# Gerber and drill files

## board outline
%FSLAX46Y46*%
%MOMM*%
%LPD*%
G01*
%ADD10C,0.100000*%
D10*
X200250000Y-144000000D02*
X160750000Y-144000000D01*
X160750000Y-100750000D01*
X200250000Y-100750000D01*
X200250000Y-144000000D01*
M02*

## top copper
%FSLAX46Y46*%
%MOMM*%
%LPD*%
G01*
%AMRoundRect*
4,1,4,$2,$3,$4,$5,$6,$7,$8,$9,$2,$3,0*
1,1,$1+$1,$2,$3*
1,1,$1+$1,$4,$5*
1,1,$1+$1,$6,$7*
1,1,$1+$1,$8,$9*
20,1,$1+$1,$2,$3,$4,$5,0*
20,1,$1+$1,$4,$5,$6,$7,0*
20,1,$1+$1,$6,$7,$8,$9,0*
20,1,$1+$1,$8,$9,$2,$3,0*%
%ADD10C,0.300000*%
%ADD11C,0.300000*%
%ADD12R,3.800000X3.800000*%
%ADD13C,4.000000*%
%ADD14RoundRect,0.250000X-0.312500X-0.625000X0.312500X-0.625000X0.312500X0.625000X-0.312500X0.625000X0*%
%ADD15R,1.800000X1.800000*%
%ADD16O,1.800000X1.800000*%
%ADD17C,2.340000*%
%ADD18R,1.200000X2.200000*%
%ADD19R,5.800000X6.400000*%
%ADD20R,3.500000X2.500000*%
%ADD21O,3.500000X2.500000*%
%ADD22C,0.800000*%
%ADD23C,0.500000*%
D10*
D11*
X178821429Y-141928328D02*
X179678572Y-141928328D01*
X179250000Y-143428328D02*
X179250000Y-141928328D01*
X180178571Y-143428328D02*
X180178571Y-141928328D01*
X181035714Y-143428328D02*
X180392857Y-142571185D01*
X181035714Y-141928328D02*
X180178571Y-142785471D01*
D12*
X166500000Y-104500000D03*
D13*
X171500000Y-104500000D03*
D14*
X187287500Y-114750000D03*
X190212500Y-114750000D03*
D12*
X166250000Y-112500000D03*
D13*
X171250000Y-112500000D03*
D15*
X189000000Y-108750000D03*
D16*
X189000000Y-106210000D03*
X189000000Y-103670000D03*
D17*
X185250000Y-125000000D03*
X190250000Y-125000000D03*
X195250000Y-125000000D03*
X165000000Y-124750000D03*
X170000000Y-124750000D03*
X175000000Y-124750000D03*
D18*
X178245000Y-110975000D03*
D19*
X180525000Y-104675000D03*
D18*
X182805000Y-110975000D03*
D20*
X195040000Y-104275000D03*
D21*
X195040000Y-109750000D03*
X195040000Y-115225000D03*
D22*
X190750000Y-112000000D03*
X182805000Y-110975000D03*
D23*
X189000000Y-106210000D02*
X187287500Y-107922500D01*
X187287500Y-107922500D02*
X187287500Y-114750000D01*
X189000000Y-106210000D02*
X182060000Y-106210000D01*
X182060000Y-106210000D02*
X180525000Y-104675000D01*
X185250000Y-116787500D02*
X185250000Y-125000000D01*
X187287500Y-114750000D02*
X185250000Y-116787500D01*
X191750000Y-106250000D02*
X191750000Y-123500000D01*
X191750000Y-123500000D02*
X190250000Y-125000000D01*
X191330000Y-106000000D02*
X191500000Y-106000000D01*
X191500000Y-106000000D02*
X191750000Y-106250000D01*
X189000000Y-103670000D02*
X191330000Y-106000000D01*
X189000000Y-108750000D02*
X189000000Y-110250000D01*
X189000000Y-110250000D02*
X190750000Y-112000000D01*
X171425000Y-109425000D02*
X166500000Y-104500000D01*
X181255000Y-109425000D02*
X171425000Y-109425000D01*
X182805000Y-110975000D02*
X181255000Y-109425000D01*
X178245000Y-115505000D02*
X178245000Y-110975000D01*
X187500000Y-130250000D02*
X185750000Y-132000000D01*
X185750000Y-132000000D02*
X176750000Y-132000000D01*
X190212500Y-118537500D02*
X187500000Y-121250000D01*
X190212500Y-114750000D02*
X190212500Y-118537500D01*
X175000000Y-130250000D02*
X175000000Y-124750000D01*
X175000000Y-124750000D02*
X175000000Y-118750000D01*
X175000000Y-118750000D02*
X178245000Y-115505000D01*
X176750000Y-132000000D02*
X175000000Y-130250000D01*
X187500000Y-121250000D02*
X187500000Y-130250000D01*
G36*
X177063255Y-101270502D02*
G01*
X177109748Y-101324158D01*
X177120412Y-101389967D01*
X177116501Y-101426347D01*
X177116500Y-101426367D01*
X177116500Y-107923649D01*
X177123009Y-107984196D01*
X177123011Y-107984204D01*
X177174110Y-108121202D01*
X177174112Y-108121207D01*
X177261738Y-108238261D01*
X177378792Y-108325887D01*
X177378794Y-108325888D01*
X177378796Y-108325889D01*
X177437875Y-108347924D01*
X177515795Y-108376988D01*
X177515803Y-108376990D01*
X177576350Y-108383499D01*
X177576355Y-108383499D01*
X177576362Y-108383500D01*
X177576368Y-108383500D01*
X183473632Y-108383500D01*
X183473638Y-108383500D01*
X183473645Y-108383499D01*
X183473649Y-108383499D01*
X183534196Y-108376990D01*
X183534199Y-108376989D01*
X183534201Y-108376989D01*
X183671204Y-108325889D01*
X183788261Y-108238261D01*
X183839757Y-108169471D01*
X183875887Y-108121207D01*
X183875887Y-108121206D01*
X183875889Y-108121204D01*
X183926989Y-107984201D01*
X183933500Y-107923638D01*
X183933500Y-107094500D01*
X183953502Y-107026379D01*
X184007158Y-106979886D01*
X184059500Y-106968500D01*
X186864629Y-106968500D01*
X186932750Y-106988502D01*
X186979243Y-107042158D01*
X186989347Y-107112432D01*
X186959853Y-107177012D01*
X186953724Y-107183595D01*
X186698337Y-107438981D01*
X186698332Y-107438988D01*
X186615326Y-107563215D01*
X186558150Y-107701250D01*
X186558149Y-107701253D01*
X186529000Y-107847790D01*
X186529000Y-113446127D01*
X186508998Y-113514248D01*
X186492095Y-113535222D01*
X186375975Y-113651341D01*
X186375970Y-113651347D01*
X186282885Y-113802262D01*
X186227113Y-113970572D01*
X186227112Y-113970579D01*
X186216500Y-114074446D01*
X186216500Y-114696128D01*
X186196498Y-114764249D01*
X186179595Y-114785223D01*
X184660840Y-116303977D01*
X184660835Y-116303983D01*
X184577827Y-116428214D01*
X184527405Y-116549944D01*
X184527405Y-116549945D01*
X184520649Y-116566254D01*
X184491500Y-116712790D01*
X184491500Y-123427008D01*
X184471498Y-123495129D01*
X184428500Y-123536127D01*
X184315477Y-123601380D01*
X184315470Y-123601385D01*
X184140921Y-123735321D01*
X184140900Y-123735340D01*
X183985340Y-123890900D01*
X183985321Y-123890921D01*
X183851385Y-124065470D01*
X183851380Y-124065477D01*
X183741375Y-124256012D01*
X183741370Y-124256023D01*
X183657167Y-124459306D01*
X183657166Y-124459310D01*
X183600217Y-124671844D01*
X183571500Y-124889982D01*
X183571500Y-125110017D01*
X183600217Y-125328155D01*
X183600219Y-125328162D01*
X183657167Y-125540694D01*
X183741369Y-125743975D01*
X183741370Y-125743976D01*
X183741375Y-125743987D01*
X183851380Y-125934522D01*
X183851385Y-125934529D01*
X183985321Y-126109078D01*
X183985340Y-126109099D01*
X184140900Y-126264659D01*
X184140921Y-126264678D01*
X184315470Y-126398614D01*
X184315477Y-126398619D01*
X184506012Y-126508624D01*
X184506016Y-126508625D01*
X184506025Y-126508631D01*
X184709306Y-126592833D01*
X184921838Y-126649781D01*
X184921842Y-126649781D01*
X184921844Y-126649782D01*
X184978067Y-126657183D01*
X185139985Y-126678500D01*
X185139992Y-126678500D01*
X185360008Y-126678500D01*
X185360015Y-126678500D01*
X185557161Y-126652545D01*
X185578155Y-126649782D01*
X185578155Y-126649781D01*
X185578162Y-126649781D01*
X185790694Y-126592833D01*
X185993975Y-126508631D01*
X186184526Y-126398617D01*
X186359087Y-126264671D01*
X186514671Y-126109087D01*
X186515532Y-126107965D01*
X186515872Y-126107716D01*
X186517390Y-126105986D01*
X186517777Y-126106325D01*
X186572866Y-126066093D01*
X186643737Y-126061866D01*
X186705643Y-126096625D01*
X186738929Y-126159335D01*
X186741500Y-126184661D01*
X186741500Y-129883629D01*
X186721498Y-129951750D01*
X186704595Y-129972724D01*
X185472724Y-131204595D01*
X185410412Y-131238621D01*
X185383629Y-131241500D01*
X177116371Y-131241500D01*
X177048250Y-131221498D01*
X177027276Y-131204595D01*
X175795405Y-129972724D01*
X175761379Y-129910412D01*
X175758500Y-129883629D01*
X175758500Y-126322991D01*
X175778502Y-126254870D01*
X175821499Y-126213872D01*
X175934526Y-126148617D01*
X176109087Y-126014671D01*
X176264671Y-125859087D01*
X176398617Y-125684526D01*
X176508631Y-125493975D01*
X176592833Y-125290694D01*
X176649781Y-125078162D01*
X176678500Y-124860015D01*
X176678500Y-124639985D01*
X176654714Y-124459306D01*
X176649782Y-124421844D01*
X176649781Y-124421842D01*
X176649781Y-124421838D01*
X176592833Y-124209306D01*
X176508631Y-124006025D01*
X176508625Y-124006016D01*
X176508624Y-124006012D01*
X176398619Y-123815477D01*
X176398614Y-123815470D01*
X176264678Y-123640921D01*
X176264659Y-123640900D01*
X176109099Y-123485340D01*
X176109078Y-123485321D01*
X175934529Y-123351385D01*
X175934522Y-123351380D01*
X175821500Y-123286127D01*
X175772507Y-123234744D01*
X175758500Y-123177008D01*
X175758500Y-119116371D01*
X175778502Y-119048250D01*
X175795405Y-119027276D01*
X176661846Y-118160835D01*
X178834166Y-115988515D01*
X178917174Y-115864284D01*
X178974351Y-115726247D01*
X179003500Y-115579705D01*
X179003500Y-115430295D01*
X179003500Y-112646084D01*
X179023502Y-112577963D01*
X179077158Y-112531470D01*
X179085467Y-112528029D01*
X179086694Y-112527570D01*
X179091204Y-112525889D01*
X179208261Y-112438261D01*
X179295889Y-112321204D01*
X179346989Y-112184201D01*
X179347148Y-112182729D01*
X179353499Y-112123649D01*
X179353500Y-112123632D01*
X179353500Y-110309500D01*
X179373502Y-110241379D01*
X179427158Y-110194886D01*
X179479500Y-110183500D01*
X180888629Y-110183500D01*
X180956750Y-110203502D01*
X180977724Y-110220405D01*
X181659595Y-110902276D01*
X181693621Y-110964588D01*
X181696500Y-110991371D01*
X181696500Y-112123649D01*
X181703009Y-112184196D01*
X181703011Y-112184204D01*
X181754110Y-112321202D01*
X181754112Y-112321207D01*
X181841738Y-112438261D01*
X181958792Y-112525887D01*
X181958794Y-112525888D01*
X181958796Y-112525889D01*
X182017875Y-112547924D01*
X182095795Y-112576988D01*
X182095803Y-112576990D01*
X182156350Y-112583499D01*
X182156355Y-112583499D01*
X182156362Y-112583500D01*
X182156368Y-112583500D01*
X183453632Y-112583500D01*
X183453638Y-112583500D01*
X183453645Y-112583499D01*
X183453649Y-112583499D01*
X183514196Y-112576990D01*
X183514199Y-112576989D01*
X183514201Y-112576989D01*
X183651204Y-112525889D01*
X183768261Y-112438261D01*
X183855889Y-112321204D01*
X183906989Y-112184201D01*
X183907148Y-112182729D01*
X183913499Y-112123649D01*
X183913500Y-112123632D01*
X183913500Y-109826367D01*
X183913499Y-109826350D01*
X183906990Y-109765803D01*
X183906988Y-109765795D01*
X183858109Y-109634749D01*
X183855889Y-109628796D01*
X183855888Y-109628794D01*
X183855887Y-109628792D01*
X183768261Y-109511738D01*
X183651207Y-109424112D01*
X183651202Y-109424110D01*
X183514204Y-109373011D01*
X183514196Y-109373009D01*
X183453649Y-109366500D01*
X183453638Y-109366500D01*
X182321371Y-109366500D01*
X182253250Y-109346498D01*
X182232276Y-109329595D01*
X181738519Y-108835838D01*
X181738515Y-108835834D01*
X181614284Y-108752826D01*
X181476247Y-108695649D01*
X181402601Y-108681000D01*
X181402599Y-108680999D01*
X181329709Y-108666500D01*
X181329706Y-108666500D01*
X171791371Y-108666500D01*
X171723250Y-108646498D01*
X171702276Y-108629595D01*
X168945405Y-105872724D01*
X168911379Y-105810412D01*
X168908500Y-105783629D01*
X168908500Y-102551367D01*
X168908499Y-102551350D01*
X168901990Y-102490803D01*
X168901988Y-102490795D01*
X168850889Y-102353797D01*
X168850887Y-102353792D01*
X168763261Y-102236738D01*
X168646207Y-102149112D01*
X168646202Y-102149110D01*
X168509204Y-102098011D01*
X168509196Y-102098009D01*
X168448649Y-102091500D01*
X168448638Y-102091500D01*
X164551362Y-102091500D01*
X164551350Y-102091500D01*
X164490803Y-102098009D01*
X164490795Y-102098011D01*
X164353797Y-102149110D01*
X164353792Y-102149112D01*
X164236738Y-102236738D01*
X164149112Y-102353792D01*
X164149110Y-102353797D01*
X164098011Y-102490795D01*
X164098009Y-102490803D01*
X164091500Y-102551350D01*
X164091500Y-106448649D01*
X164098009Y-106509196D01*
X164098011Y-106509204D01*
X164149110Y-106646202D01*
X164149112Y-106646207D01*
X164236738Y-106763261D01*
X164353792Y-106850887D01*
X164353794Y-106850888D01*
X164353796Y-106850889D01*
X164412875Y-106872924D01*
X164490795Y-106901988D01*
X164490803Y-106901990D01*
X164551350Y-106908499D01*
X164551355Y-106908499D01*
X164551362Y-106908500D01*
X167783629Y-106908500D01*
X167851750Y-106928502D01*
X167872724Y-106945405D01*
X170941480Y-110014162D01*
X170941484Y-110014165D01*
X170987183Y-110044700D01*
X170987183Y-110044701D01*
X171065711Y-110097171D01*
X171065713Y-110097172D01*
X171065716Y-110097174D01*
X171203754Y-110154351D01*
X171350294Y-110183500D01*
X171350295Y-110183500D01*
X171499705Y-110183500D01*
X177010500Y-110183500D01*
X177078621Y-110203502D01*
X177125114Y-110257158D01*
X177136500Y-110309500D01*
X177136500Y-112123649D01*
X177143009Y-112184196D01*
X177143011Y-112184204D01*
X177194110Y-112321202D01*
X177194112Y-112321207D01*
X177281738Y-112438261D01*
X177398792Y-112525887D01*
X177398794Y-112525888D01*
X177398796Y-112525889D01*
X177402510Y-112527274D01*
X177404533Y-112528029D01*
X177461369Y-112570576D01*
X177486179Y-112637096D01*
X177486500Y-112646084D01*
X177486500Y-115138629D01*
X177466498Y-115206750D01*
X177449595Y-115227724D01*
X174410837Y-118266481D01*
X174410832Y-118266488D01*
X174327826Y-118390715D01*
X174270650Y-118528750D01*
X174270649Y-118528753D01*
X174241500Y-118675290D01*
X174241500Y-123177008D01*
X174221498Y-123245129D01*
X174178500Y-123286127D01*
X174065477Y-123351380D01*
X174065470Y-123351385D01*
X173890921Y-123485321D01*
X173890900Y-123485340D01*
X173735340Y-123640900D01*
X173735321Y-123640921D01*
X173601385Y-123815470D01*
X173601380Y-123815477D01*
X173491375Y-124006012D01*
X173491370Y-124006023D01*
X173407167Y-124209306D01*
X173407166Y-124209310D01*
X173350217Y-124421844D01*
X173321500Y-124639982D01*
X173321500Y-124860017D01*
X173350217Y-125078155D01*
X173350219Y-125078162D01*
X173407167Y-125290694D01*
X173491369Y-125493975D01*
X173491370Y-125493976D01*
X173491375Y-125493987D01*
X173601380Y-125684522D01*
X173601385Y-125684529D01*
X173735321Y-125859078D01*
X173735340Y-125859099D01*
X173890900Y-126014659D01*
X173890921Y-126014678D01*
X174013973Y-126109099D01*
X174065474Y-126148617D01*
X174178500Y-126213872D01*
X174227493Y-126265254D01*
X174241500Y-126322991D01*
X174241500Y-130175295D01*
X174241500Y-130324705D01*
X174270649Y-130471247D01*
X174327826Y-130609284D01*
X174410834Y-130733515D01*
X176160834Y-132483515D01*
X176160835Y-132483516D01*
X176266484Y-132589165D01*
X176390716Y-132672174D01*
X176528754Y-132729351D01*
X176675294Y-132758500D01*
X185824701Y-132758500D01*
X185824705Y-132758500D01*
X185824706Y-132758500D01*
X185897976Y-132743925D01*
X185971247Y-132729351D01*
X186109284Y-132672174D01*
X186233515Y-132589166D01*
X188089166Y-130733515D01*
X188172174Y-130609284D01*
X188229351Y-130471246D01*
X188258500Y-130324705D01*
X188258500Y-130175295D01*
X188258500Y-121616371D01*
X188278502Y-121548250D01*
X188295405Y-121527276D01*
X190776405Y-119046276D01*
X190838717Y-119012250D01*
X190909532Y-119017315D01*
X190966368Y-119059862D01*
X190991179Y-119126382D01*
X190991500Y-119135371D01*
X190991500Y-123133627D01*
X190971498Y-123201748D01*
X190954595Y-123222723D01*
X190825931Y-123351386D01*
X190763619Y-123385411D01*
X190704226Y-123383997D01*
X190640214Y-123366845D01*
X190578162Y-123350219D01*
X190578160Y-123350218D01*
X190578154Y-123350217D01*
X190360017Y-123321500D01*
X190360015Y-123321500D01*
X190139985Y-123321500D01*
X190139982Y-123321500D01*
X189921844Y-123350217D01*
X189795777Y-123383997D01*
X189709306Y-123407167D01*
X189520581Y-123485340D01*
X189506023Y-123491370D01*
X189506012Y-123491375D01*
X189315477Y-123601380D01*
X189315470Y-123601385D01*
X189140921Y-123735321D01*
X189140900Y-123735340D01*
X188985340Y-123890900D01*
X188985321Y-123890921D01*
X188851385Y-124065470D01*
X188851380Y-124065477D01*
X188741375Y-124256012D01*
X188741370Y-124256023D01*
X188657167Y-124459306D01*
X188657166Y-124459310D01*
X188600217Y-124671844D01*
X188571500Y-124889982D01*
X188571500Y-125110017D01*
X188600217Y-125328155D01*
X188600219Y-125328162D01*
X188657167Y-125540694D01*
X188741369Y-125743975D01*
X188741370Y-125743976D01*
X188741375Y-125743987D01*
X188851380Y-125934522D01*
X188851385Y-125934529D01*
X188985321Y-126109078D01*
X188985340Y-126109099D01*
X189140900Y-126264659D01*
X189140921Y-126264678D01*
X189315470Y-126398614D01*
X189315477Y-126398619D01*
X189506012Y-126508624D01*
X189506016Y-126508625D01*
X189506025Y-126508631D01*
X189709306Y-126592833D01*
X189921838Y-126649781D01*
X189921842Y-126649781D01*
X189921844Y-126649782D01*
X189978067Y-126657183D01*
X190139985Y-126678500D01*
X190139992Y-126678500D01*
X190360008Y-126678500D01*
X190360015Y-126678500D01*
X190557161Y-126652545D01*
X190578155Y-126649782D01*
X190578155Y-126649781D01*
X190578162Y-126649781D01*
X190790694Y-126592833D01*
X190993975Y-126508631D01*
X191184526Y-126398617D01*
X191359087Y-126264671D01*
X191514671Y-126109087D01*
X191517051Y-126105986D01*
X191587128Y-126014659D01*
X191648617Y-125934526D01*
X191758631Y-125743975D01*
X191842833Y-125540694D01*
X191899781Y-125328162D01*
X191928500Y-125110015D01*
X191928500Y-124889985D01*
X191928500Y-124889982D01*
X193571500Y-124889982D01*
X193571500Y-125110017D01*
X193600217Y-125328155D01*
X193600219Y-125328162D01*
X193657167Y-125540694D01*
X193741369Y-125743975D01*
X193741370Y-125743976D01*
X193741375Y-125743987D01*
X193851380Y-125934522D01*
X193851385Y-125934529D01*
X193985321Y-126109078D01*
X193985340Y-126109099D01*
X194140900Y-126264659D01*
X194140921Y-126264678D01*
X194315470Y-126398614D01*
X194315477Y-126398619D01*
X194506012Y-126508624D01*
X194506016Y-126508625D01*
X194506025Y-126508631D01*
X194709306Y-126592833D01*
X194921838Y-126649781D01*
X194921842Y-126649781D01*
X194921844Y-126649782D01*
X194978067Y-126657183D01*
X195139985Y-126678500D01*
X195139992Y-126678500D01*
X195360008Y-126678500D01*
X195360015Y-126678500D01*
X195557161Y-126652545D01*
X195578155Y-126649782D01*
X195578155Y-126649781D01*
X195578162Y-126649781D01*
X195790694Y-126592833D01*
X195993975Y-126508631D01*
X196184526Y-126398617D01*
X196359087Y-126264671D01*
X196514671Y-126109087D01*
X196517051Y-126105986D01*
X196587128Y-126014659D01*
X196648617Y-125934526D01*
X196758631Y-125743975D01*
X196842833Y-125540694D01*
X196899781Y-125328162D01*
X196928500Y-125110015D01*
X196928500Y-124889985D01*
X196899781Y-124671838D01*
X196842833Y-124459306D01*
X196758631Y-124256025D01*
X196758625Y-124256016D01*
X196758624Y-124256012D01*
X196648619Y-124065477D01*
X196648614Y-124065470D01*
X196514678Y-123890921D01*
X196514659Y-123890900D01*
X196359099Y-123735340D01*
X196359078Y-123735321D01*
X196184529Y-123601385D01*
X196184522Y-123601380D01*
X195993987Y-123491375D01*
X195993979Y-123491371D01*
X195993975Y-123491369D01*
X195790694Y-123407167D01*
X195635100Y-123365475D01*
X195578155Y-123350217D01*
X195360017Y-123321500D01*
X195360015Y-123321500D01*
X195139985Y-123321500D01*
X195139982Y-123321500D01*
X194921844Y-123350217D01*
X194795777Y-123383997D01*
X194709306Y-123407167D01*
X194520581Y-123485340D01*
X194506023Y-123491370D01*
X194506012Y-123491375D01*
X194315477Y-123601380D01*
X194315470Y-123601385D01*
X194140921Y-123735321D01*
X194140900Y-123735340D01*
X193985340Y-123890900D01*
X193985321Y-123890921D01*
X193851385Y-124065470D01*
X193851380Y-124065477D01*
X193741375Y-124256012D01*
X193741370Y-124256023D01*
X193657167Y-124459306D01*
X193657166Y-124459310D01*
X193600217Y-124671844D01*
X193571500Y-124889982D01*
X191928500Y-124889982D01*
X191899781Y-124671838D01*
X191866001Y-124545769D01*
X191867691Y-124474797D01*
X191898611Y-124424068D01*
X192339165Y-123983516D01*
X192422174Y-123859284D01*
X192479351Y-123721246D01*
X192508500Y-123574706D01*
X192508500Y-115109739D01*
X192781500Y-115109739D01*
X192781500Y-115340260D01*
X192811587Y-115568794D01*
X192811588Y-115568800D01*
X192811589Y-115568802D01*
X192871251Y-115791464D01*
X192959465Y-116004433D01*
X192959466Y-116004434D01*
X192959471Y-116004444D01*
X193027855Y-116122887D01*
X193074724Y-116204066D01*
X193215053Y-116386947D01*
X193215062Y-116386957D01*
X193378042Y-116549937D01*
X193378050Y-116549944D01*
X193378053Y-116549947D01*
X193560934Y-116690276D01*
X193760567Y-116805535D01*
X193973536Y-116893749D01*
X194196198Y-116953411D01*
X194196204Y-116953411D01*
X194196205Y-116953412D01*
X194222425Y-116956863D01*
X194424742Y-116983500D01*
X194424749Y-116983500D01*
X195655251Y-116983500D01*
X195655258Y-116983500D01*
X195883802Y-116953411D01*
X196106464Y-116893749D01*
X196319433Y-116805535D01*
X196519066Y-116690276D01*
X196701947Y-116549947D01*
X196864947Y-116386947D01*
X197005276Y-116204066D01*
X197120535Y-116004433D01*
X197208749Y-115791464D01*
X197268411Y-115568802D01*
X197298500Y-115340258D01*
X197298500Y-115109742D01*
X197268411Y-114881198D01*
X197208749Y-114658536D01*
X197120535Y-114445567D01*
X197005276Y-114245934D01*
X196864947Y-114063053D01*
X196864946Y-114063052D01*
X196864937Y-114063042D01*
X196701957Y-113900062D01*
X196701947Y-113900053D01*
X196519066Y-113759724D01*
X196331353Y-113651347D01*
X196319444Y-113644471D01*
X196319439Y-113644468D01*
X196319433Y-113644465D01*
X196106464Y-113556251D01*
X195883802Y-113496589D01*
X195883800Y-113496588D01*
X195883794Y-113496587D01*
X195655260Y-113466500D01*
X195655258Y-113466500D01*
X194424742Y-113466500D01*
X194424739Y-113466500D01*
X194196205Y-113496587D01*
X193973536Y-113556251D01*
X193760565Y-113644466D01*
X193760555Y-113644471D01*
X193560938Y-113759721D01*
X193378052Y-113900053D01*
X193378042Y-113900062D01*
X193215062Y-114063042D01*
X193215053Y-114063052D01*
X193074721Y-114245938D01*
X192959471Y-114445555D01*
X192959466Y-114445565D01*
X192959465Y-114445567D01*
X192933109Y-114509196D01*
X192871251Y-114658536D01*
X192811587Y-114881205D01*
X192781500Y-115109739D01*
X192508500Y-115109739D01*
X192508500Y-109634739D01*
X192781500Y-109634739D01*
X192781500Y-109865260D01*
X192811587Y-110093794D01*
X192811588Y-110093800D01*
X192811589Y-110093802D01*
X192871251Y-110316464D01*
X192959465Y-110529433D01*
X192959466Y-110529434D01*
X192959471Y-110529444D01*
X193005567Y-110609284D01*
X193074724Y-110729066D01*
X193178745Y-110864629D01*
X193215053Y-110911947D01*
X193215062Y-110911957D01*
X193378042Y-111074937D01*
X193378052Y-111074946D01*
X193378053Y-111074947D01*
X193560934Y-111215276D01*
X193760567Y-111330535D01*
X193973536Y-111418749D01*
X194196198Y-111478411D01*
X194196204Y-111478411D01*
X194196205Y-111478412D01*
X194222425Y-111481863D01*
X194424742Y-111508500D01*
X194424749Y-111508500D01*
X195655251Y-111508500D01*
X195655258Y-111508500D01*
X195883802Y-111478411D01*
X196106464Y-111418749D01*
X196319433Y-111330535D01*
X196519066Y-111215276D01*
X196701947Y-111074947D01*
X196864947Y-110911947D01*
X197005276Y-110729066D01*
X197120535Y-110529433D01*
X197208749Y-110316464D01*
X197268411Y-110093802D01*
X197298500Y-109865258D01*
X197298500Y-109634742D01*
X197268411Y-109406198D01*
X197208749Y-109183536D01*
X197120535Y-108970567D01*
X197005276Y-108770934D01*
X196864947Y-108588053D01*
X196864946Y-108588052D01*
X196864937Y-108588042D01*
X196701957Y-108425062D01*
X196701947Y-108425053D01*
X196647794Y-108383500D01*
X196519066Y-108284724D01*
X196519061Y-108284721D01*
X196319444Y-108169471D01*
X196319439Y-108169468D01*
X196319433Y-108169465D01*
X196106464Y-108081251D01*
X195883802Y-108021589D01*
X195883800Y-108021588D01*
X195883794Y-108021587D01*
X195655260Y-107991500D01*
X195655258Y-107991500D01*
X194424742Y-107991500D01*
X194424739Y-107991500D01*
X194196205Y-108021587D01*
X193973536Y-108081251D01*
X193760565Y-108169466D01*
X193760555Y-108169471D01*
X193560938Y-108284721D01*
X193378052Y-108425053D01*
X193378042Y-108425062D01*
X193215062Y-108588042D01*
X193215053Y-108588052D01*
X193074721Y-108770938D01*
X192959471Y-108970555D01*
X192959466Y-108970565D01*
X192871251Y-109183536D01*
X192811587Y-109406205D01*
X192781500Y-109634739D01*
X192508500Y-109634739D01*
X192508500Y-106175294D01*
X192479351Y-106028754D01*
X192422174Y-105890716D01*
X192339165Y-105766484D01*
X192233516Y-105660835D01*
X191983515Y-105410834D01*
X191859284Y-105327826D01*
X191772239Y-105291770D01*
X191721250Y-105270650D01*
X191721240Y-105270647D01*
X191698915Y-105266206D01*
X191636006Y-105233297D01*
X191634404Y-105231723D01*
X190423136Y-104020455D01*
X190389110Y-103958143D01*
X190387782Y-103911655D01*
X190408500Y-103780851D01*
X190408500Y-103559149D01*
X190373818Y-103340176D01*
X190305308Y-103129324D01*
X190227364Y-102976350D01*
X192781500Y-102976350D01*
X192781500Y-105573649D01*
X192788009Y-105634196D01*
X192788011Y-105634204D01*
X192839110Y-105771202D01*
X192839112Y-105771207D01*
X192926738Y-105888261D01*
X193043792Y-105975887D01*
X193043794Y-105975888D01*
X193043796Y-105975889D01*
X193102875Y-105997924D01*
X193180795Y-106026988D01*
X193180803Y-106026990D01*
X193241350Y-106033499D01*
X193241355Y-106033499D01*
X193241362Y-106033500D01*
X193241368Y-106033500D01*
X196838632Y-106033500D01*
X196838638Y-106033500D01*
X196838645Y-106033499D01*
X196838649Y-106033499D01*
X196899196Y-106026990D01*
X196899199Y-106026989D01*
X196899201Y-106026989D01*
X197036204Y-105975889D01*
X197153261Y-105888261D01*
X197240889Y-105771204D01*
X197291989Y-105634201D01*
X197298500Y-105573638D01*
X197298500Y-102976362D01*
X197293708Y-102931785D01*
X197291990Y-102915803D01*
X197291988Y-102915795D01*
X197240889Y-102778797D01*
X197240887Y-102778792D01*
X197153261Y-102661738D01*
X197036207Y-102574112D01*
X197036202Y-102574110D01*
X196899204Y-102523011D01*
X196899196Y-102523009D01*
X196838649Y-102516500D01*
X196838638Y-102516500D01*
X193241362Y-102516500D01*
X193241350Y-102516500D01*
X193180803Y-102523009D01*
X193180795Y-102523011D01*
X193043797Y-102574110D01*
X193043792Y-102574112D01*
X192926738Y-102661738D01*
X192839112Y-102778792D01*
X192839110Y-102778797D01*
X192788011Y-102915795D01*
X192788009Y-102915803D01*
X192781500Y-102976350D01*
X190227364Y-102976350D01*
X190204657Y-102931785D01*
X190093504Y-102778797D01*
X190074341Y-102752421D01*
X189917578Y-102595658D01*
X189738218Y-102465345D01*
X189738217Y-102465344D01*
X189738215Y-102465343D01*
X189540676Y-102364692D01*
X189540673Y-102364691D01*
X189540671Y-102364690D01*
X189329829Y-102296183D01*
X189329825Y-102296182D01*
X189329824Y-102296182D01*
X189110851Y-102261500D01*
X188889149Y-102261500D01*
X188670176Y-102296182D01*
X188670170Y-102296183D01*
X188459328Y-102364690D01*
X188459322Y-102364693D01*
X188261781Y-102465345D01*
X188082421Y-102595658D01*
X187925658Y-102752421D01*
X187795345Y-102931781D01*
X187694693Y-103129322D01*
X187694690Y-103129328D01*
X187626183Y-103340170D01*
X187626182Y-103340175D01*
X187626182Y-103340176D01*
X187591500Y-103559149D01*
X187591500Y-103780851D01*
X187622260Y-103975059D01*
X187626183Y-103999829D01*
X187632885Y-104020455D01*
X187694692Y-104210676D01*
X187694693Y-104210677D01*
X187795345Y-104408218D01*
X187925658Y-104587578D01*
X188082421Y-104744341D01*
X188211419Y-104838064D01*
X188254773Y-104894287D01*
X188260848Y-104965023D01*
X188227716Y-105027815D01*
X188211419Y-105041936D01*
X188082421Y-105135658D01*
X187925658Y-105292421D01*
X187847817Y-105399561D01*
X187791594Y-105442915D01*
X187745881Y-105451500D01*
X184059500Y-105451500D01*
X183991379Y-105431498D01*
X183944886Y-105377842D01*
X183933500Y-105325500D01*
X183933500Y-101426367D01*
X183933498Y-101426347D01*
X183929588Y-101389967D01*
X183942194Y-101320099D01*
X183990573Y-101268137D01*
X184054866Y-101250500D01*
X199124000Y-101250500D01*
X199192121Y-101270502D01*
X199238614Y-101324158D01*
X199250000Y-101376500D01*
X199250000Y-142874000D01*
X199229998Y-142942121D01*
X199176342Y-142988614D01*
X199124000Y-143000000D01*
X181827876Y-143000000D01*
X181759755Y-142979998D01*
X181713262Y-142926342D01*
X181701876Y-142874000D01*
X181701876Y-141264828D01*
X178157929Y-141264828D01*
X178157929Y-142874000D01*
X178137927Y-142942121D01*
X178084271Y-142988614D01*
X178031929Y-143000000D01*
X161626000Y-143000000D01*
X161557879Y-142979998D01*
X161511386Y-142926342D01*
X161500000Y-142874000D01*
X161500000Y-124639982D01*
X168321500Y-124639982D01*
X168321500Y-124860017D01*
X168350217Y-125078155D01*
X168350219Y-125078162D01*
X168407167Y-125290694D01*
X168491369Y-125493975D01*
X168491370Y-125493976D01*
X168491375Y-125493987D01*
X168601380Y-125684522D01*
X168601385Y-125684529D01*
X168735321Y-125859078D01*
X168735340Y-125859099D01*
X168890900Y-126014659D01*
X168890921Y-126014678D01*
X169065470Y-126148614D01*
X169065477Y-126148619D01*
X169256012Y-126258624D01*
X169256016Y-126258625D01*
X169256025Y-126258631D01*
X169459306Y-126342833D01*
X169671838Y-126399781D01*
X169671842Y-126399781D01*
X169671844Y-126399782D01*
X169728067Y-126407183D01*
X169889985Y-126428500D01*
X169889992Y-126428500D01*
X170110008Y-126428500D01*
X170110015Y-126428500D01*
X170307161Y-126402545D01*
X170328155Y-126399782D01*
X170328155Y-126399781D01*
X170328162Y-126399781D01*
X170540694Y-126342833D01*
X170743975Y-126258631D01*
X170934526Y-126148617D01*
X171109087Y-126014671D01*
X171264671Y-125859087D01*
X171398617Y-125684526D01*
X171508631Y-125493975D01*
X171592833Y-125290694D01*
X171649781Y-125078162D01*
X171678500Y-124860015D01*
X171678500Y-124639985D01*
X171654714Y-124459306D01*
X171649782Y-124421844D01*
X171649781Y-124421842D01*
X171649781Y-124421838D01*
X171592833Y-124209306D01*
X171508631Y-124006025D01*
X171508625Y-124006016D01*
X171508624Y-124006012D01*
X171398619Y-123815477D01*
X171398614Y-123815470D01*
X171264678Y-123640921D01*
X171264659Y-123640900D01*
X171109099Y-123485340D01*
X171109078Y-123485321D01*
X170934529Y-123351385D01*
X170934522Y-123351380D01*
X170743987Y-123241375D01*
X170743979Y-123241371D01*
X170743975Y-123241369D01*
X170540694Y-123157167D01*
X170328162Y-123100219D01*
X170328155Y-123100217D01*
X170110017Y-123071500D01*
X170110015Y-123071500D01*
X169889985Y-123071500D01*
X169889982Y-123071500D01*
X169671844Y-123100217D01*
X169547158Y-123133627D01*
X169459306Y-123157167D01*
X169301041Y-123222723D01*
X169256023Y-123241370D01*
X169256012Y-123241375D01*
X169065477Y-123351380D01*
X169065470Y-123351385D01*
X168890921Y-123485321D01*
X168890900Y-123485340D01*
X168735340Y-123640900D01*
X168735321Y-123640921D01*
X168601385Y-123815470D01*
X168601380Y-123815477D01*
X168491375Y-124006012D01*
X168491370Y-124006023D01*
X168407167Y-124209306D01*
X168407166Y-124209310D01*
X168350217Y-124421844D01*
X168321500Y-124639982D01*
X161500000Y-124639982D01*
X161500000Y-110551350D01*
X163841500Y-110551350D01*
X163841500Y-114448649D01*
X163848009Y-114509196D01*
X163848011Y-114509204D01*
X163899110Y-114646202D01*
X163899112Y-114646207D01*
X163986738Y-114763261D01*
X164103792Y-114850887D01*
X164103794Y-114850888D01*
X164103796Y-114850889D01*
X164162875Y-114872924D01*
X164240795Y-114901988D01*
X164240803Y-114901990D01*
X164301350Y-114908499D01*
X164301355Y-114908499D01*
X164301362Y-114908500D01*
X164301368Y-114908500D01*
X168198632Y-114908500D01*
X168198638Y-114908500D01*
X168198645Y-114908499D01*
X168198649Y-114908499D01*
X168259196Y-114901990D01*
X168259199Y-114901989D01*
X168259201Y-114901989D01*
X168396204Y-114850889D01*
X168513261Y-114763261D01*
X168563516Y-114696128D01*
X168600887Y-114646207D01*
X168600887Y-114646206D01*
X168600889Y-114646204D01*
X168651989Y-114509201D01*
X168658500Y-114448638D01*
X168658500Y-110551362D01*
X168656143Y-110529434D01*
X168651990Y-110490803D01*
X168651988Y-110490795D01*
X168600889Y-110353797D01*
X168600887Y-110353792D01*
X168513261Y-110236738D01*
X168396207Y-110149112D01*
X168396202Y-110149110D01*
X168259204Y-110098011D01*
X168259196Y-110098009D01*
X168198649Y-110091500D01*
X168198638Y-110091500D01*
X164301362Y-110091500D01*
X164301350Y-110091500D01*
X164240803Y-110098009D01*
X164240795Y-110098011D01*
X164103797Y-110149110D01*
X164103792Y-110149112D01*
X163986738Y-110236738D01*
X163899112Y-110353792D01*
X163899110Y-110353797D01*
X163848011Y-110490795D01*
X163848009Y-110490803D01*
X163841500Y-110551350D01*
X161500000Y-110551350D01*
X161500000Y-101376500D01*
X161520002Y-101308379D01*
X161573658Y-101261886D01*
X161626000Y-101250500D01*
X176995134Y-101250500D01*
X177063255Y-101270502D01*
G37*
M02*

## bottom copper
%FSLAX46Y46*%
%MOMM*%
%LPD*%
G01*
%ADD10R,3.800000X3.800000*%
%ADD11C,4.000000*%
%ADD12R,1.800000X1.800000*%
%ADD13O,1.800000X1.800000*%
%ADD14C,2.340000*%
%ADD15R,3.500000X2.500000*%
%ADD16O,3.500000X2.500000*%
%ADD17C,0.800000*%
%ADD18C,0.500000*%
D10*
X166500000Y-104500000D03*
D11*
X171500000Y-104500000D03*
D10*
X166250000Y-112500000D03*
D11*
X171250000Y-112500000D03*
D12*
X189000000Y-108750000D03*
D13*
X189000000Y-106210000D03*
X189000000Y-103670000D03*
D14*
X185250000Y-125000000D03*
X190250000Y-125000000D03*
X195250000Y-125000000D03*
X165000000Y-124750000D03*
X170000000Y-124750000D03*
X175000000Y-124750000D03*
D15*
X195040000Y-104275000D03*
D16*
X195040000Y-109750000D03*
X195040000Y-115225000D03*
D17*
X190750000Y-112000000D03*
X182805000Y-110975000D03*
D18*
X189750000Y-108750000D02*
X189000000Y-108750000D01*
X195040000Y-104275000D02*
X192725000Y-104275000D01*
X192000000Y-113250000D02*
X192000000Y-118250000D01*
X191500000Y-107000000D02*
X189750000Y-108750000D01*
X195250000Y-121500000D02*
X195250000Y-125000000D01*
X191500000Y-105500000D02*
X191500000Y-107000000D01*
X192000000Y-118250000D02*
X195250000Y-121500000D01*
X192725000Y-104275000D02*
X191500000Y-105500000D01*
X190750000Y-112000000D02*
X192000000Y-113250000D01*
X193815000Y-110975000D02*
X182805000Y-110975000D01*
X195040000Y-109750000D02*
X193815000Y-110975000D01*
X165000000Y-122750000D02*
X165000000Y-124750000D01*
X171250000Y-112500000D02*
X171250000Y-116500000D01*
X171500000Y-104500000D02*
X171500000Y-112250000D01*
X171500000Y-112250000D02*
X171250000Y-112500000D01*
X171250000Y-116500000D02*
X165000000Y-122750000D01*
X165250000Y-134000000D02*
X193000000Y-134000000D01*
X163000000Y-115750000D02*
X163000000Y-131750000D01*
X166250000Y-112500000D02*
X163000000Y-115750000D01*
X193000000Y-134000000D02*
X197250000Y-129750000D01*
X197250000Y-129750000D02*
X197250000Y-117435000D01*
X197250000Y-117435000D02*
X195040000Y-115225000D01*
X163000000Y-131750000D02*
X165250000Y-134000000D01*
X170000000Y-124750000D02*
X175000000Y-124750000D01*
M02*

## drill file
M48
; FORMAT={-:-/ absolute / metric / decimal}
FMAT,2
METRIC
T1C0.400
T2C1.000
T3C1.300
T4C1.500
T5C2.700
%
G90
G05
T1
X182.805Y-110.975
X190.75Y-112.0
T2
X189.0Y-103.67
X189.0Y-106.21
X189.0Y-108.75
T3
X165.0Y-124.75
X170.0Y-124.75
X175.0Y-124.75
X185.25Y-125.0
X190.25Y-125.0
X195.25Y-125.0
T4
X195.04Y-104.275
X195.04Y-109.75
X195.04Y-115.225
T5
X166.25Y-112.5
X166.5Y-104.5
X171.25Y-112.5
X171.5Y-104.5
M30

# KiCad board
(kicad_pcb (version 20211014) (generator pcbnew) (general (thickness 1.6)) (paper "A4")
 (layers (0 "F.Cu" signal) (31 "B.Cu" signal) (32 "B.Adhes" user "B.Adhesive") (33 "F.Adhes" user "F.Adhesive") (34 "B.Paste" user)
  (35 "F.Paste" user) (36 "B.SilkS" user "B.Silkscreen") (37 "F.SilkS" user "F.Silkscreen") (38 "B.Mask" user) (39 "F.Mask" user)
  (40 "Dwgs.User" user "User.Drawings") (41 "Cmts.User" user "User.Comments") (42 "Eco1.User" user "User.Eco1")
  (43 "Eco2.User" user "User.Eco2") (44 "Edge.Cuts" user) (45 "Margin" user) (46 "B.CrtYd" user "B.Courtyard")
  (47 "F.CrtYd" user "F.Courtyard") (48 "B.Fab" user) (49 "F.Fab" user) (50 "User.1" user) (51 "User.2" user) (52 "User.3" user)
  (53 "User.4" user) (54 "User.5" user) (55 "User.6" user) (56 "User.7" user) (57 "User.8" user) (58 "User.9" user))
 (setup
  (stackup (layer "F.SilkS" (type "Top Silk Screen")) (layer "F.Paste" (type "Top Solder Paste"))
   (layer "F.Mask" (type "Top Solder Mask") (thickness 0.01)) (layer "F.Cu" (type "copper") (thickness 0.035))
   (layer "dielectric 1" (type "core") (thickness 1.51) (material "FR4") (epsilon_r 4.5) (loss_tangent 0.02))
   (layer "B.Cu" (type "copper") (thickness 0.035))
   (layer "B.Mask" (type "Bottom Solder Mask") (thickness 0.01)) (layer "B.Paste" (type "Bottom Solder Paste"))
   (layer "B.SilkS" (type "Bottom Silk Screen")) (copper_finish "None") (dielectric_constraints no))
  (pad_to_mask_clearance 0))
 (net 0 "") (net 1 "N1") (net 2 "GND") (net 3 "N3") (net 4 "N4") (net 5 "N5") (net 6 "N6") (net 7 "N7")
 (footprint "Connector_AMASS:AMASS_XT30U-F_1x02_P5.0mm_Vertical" (layer "F.Cu") (at 166.5 104.5)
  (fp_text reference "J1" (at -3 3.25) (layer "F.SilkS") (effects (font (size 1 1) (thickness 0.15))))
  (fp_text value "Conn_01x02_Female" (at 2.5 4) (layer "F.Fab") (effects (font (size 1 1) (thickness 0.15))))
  (pad "1" thru_hole rect (at 0 0) (size 3.8 3.8) (drill 2.7) (layers *.Cu *.Mask) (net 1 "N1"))
  (pad "2" thru_hole circle (at 5 0) (size 4 4) (drill 2.7) (layers *.Cu *.Mask) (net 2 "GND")))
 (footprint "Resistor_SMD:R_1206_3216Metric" (layer "F.Cu") (at 188.75 114.75)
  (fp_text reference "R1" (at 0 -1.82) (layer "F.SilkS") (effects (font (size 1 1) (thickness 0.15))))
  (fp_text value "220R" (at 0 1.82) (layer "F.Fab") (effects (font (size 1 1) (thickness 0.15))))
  (pad "1" smd roundrect (at -1.4625 0) (size 1.125 1.75) (layers "F.Cu" "F.Paste" "F.Mask") (roundrect_rratio 0.2222222222) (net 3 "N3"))
  (pad "2" smd roundrect (at 1.4625 0) (size 1.125 1.75) (layers "F.Cu" "F.Paste" "F.Mask") (roundrect_rratio 0.2222222222) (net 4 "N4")))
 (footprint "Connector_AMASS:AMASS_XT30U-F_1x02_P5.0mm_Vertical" (layer "F.Cu") (at 166.25 112.5)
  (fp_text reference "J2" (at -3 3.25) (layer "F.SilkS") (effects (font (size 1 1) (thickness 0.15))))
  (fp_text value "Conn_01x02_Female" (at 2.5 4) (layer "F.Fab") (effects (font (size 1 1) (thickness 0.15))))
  (pad "1" thru_hole rect (at 0 0) (size 3.8 3.8) (drill 2.7) (layers *.Cu *.Mask) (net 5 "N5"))
  (pad "2" thru_hole circle (at 5 0) (size 4 4) (drill 2.7) (layers *.Cu *.Mask) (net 2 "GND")))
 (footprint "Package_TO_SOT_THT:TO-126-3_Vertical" (layer "F.Cu") (at 189 108.75 90)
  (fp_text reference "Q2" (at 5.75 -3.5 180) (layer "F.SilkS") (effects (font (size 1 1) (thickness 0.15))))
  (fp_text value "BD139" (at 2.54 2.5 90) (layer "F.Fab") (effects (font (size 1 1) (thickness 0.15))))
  (pad "1" thru_hole rect (at 0 0 90) (size 1.8 1.8) (drill 1) (layers *.Cu *.Mask) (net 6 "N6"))
  (pad "2" thru_hole oval (at 2.54 0 90) (size 1.8 1.8) (drill 1) (layers *.Cu *.Mask) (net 3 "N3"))
  (pad "3" thru_hole oval (at 5.08 0 90) (size 1.8 1.8) (drill 1) (layers *.Cu *.Mask) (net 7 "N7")))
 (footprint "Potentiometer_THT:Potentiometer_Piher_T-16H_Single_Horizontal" (layer "F.Cu") (at 185.25 125 -90)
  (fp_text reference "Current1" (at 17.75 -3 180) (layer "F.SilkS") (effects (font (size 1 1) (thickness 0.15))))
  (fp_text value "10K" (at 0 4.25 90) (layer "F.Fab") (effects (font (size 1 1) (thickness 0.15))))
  (pad "1" thru_hole circle (at 0 0 270) (size 2.34 2.34) (drill 1.3) (layers *.Cu *.Mask) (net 3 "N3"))
  (pad "2" thru_hole circle (at 0 -5 270) (size 2.34 2.34) (drill 1.3) (layers *.Cu *.Mask) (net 7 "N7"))
  (pad "3" thru_hole circle (at 0 -10 270) (size 2.34 2.34) (drill 1.3) (layers *.Cu *.Mask) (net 6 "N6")))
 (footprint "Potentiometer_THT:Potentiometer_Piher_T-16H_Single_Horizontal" (layer "F.Cu") (at 165 124.75 -90)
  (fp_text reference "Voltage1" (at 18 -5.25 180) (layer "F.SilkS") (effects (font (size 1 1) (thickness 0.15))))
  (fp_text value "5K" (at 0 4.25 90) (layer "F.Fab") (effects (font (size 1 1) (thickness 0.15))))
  (pad "1" thru_hole circle (at 0 0 270) (size 2.34 2.34) (drill 1.3) (layers *.Cu *.Mask) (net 2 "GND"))
  (pad "2" thru_hole circle (at 0 -5 270) (size 2.34 2.34) (drill 1.3) (layers *.Cu *.Mask) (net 4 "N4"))
  (pad "3" thru_hole circle (at 0 -10 270) (size 2.34 2.34) (drill 1.3) (layers *.Cu *.Mask) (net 4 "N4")))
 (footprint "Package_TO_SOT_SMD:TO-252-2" (layer "F.Cu") (at 180.525 106.775 90)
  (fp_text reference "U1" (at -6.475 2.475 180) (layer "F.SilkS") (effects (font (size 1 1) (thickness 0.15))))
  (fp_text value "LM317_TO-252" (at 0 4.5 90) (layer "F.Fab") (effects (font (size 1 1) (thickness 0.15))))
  (pad "" smd rect (at 0.425 1.525 90) (size 3.05 2.75) (layers "F.Paste"))
  (pad "" smd rect (at 0.425 -1.525 90) (size 3.05 2.75) (layers "F.Paste"))
  (pad "" smd rect (at 3.775 -1.525 90) (size 3.05 2.75) (layers "F.Paste"))
  (pad "" smd rect (at 3.775 1.525 90) (size 3.05 2.75) (layers "F.Paste"))
  (pad "1" smd rect (at -4.2 -2.28 90) (size 2.2 1.2) (layers "F.Cu" "F.Paste" "F.Mask") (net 4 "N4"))
  (pad "2" smd rect (at 2.1 0 90) (size 6.4 5.8) (layers "F.Cu" "F.Mask") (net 3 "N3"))
  (pad "3" smd rect (at -4.2 2.28 90) (size 2.2 1.2) (layers "F.Cu" "F.Paste" "F.Mask") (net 1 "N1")))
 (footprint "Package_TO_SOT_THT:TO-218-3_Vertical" (layer "F.Cu") (at 195.04 104.275 -90)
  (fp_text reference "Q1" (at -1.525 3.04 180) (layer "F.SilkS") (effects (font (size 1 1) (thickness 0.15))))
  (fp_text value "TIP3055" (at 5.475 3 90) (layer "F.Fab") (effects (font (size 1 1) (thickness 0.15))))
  (pad "1" thru_hole rect (at 0 0 270) (size 2.5 3.5) (drill 1.5) (layers *.Cu *.Mask) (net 6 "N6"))
  (pad "2" thru_hole oval (at 5.475 0 270) (size 2.5 3.5) (drill 1.5) (layers *.Cu *.Mask) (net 1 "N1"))
  (pad "3" thru_hole oval (at 10.95 0 270) (size 2.5 3.5) (drill 1.5) (layers *.Cu *.Mask) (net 5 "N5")))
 (gr_poly (pts (xy 200.25 144) (xy 160.75 144) (xy 160.75 100.75) (xy 200.25 100.75)) (layer "Edge.Cuts") (width 0.1) (fill none))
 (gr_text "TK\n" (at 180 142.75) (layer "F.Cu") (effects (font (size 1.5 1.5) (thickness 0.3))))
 (segment (start 189 106.21) (end 187.2875 107.9225) (width 0.5) (layer "F.Cu") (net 3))
 (segment (start 187.2875 107.9225) (end 187.2875 114.75) (width 0.5) (layer "F.Cu") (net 3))
 (segment (start 189 106.21) (end 182.06 106.21) (width 0.5) (layer "F.Cu") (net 3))
 (segment (start 182.06 106.21) (end 180.525 104.675) (width 0.5) (layer "F.Cu") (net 3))
 (segment (start 185.25 116.7875) (end 185.25 125) (width 0.5) (layer "F.Cu") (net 3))
 (segment (start 187.2875 114.75) (end 185.25 116.7875) (width 0.5) (layer "F.Cu") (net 3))
 (segment (start 191.75 106.25) (end 191.75 123.5) (width 0.5) (layer "F.Cu") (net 7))
 (segment (start 191.75 123.5) (end 190.25 125) (width 0.5) (layer "F.Cu") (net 7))
 (segment (start 191.33 106) (end 191.5 106) (width 0.5) (layer "F.Cu") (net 7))
 (segment (start 191.5 106) (end 191.75 106.25) (width 0.5) (layer "F.Cu") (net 7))
 (segment (start 189 103.67) (end 191.33 106) (width 0.5) (layer "F.Cu") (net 7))
 (segment (start 189 108.75) (end 189 110.25) (width 0.5) (layer "F.Cu") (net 6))
 (segment (start 189 110.25) (end 190.75 112) (width 0.5) (layer "F.Cu") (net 6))
 (via (at 190.75 112) (size 0.8) (drill 0.4) (layers "F.Cu" "B.Cu") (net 6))
 (segment (start 189.75 108.75) (end 189 108.75) (width 0.5) (layer "B.Cu") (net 6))
 (segment (start 195.04 104.275) (end 192.725 104.275) (width 0.5) (layer "B.Cu") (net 6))
 (segment (start 192 113.25) (end 192 118.25) (width 0.5) (layer "B.Cu") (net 6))
 (segment (start 191.5 107) (end 189.75 108.75) (width 0.5) (layer "B.Cu") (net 6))
 (segment (start 195.25 121.5) (end 195.25 125) (width 0.5) (layer "B.Cu") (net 6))
 (segment (start 191.5 105.5) (end 191.5 107) (width 0.5) (layer "B.Cu") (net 6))
 (segment (start 192 118.25) (end 195.25 121.5) (width 0.5) (layer "B.Cu") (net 6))
 (segment (start 192.725 104.275) (end 191.5 105.5) (width 0.5) (layer "B.Cu") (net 6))
 (segment (start 190.75 112) (end 192 113.25) (width 0.5) (layer "B.Cu") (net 6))
 (segment (start 171.425 109.425) (end 166.5 104.5) (width 0.5) (layer "F.Cu") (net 1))
 (segment (start 181.255 109.425) (end 171.425 109.425) (width 0.5) (layer "F.Cu") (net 1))
 (segment (start 182.805 110.975) (end 181.255 109.425) (width 0.5) (layer "F.Cu") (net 1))
 (via (at 182.805 110.975) (size 0.8) (drill 0.4) (layers "F.Cu" "B.Cu") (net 1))
 (segment (start 193.815 110.975) (end 182.805 110.975) (width 0.5) (layer "B.Cu") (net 1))
 (segment (start 195.04 109.75) (end 193.815 110.975) (width 0.5) (layer "B.Cu") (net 1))
 (segment (start 165 122.75) (end 165 124.75) (width 0.5) (layer "B.Cu") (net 2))
 (segment (start 171.25 112.5) (end 171.25 116.5) (width 0.5) (layer "B.Cu") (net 2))
 (segment (start 171.5 104.5) (end 171.5 112.25) (width 0.5) (layer "B.Cu") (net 2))
 (segment (start 171.5 112.25) (end 171.25 112.5) (width 0.5) (layer "B.Cu") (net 2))
 (segment (start 171.25 116.5) (end 165 122.75) (width 0.5) (layer "B.Cu") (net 2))
 (segment (start 165.25 134) (end 193 134) (width 0.5) (layer "B.Cu") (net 5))
 (segment (start 163 115.75) (end 163 131.75) (width 0.5) (layer "B.Cu") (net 5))
 (segment (start 166.25 112.5) (end 163 115.75) (width 0.5) (layer "B.Cu") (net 5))
 (segment (start 193 134) (end 197.25 129.75) (width 0.5) (layer "B.Cu") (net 5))
 (segment (start 197.25 129.75) (end 197.25 117.435) (width 0.5) (layer "B.Cu") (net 5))
 (segment (start 197.25 117.435) (end 195.04 115.225) (width 0.5) (layer "B.Cu") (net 5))
 (segment (start 163 131.75) (end 165.25 134) (width 0.5) (layer "B.Cu") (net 5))
 (segment (start 178.245 115.505) (end 178.245 110.975) (width 0.5) (layer "F.Cu") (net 4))
 (segment (start 187.5 130.25) (end 185.75 132) (width 0.5) (layer "F.Cu") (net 4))
 (segment (start 185.75 132) (end 176.75 132) (width 0.5) (layer "F.Cu") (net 4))
 (segment (start 190.2125 118.5375) (end 187.5 121.25) (width 0.5) (layer "F.Cu") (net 4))
 (segment (start 190.2125 114.75) (end 190.2125 118.5375) (width 0.5) (layer "F.Cu") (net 4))
 (segment (start 175 130.25) (end 175 124.75) (width 0.5) (layer "F.Cu") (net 4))
 (segment (start 175 124.75) (end 175 118.75) (width 0.5) (layer "F.Cu") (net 4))
 (segment (start 175 118.75) (end 178.245 115.505) (width 0.5) (layer "F.Cu") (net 4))
 (segment (start 176.75 132) (end 175 130.25) (width 0.5) (layer "F.Cu") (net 4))
 (segment (start 187.5 121.25) (end 187.5 130.25) (width 0.5) (layer "F.Cu") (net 4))
 (segment (start 170 124.75) (end 175 124.75) (width 0.5) (layer "B.Cu") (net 4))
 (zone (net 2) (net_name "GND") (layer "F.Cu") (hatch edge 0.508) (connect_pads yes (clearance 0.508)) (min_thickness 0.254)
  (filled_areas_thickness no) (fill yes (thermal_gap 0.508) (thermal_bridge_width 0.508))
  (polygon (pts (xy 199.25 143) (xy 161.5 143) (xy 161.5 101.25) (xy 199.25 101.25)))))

